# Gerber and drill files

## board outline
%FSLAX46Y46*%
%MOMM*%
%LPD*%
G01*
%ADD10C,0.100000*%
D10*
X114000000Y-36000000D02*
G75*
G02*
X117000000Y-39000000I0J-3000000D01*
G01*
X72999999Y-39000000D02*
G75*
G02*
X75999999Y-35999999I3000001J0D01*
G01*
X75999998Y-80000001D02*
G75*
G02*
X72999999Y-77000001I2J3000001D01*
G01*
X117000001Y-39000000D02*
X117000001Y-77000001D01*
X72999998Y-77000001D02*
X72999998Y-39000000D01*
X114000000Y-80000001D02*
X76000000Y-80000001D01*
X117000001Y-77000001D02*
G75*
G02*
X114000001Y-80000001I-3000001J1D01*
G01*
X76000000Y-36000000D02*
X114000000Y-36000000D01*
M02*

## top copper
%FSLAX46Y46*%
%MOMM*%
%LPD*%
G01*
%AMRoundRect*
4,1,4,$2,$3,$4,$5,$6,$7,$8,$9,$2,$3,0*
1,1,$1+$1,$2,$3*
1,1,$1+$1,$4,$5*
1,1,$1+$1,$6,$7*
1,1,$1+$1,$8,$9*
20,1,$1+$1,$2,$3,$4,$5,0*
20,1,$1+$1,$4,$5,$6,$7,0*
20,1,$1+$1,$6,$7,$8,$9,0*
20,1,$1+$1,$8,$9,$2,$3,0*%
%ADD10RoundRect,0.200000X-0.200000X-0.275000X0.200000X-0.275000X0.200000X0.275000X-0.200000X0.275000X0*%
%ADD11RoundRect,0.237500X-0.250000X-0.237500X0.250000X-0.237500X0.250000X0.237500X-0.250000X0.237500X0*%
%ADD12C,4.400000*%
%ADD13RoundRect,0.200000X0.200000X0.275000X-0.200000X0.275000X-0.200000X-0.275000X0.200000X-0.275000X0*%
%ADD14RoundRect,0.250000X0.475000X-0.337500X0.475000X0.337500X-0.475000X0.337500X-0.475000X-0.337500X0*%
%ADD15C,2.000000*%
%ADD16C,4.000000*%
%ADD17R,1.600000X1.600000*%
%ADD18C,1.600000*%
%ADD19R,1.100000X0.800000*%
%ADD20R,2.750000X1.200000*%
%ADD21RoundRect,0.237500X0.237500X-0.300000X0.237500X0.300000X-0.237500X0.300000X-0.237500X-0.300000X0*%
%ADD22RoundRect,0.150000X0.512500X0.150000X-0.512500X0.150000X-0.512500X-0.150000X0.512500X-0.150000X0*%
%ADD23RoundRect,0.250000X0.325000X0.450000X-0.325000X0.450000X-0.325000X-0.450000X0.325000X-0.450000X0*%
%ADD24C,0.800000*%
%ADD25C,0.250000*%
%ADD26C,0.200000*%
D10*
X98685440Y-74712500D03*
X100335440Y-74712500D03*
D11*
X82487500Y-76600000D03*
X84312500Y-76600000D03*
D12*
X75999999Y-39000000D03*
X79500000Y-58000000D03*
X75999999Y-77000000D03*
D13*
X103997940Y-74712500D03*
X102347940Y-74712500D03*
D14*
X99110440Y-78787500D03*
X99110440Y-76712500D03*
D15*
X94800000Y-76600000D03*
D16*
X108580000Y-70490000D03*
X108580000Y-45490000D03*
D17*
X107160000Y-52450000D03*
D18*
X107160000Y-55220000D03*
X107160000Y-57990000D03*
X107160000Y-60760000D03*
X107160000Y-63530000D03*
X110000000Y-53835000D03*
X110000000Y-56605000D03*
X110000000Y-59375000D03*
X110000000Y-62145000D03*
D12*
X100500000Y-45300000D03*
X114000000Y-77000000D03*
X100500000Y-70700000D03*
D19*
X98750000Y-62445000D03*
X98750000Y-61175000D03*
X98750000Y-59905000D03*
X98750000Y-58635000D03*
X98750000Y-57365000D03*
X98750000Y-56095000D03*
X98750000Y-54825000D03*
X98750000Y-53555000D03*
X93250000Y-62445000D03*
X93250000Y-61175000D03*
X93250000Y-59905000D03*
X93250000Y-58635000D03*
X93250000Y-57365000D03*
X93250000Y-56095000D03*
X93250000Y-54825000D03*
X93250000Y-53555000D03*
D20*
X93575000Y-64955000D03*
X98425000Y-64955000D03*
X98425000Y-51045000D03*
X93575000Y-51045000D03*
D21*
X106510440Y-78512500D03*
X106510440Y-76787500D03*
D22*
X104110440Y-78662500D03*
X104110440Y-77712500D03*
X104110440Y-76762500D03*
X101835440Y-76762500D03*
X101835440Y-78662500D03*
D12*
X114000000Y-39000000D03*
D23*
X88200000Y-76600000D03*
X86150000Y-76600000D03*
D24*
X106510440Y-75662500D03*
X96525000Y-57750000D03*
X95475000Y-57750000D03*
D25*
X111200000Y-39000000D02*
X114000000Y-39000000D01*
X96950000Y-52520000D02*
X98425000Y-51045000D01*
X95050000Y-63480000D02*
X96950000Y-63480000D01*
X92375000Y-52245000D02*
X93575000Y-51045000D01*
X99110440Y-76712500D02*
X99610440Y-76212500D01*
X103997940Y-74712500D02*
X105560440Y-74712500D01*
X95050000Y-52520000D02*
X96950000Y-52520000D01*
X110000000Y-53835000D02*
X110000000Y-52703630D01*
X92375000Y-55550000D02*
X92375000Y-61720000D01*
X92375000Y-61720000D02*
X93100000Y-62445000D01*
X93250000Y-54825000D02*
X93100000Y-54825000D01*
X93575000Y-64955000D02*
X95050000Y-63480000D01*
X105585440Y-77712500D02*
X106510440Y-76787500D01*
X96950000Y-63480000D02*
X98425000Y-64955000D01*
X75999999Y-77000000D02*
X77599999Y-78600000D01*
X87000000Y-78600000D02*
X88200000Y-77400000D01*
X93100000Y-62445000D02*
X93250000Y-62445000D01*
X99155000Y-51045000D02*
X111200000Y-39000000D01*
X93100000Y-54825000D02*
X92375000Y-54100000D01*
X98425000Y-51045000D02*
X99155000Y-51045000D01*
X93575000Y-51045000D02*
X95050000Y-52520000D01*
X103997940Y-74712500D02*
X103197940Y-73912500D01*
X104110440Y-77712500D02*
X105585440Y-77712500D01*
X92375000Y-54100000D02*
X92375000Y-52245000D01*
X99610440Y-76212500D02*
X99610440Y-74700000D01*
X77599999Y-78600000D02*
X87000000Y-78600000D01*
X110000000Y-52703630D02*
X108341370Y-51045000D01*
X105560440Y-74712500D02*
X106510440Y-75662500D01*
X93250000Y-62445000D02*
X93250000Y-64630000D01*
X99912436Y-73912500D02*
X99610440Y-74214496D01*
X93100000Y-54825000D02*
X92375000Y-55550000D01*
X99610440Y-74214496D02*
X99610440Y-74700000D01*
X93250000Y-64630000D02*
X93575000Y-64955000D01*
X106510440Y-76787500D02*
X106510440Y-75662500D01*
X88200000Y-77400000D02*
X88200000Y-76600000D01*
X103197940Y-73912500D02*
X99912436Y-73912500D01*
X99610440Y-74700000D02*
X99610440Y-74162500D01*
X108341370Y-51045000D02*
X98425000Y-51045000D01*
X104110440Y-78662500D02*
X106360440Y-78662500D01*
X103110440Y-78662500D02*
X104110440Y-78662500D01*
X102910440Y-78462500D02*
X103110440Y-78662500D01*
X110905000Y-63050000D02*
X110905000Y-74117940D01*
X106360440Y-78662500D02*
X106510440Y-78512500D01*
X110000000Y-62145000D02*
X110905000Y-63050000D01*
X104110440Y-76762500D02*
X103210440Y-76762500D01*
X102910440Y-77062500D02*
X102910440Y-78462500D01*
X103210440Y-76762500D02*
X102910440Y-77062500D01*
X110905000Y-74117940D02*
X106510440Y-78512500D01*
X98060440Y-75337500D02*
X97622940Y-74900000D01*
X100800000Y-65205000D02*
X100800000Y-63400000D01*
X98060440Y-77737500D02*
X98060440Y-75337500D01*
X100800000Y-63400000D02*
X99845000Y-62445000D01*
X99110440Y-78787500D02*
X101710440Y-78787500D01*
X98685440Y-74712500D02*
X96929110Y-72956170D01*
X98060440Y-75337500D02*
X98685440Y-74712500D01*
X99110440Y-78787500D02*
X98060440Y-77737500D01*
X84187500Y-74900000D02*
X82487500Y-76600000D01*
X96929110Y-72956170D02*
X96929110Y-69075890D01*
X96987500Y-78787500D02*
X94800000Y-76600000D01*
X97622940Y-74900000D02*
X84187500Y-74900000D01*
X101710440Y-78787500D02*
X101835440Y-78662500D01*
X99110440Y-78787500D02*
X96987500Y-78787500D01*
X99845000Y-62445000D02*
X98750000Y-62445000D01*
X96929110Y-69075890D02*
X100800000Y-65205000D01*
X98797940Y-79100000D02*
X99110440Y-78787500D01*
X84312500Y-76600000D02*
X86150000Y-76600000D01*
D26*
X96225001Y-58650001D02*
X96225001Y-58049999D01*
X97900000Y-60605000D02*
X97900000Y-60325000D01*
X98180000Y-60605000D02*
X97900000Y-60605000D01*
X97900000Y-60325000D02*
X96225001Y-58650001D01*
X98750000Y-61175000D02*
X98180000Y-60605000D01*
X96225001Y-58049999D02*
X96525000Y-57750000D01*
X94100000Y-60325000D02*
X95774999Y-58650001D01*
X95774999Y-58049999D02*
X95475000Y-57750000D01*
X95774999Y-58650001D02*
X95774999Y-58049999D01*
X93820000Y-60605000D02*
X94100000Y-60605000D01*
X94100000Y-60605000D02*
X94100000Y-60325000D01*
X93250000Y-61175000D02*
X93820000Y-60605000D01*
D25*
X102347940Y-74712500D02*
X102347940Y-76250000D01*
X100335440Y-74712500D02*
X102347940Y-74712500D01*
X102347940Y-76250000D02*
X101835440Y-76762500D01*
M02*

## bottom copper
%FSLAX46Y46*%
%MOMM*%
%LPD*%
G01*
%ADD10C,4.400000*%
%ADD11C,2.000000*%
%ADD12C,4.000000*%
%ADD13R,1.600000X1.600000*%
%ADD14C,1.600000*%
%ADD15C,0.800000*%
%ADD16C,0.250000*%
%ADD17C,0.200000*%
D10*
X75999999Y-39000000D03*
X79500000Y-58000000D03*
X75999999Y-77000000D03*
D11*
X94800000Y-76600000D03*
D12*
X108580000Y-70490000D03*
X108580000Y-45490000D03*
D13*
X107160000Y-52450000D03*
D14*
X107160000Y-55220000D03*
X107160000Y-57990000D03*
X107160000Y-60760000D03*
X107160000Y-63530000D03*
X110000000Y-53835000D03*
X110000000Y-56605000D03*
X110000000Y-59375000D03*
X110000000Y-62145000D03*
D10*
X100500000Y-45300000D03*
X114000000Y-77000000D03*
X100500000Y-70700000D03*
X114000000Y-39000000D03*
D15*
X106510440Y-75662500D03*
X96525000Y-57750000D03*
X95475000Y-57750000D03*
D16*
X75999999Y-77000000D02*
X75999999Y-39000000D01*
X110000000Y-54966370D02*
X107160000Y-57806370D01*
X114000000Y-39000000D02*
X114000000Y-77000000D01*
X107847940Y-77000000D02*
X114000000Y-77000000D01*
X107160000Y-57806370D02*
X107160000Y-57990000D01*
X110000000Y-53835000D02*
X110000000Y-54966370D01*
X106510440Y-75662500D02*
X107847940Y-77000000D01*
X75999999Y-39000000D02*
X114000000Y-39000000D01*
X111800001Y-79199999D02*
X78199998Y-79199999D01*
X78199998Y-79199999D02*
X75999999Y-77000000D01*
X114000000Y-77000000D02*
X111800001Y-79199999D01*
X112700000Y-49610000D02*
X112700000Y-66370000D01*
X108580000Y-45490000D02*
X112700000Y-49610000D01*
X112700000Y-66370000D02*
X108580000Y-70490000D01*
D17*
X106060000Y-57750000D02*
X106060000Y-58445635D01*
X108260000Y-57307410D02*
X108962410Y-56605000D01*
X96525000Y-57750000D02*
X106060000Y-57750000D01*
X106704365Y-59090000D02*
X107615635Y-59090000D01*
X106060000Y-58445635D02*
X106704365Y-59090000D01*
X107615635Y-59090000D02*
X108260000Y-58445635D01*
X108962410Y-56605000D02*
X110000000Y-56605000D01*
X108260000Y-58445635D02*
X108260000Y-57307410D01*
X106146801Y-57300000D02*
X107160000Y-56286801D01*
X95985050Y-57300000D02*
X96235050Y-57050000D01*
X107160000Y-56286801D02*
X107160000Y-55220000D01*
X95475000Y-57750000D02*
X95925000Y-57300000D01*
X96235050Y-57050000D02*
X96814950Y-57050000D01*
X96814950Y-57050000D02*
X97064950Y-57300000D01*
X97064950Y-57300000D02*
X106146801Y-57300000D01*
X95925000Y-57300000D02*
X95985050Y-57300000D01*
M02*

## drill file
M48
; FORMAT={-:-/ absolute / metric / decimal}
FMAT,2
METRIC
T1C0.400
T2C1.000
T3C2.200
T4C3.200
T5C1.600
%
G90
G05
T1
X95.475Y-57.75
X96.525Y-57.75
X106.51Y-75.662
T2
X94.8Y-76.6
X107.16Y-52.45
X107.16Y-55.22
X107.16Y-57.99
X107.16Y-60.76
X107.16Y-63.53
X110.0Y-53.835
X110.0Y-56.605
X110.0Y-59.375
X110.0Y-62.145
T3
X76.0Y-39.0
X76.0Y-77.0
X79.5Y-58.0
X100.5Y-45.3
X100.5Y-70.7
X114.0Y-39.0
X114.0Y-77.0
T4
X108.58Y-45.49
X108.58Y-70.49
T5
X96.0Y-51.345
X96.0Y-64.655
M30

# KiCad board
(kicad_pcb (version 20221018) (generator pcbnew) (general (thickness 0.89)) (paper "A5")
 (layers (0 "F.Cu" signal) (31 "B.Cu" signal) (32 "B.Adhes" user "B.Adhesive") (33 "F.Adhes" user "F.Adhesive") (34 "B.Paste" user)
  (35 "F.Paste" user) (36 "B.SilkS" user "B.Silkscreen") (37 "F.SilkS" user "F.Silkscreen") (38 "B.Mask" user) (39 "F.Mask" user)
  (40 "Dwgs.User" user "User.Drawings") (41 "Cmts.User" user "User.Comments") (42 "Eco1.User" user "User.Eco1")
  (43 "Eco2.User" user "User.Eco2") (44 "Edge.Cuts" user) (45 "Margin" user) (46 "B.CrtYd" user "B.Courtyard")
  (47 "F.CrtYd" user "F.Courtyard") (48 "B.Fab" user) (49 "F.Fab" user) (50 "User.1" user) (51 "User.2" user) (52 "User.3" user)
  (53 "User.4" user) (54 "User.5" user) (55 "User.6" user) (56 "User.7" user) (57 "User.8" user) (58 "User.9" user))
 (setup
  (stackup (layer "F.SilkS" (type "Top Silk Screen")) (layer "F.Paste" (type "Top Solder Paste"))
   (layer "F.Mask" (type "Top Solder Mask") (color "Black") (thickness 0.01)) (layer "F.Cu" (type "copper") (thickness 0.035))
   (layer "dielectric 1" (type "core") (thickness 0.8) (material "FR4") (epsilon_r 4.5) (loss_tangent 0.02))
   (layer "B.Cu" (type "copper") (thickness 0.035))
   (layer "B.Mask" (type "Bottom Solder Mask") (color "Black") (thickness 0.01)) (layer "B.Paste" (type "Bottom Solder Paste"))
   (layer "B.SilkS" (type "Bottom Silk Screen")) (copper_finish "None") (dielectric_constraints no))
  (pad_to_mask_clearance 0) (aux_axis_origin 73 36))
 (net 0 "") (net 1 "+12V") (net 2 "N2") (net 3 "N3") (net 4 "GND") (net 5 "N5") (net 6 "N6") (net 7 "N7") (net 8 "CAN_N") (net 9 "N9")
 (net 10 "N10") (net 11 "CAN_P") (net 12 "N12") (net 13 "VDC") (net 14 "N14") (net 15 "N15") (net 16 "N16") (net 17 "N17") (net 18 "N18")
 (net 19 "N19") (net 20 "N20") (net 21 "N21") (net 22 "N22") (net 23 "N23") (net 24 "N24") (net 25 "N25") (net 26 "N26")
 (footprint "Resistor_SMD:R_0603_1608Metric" (layer "F.Cu") (at 99.51044 74.7125)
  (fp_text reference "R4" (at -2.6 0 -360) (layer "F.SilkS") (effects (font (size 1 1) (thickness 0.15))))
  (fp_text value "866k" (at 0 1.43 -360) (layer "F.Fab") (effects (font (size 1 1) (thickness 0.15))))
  (pad "1" smd roundrect (at -0.825 0) (size 0.8 0.95) (layers "F.Cu" "F.Paste" "F.Mask") (roundrect_rratio 0.25) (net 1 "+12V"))
  (pad "2" smd roundrect (at 0.825 0) (size 0.8 0.95) (layers "F.Cu" "F.Paste" "F.Mask") (roundrect_rratio 0.25) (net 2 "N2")))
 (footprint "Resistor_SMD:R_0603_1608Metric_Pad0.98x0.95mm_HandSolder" (layer "F.Cu") (at 83.4 76.6)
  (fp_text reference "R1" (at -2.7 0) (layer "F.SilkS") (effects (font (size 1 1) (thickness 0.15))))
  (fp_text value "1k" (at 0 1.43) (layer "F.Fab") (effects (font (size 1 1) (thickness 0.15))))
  (pad "1" smd roundrect (at -0.9125 0) (size 0.975 0.95) (layers "F.Cu" "F.Paste" "F.Mask") (roundrect_rratio 0.25) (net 1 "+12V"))
  (pad "2" smd roundrect (at 0.9125 0) (size 0.975 0.95) (layers "F.Cu" "F.Paste" "F.Mask") (roundrect_rratio 0.25) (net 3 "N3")))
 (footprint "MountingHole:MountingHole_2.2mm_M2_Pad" (layer "F.Cu") (at 75.999999 39)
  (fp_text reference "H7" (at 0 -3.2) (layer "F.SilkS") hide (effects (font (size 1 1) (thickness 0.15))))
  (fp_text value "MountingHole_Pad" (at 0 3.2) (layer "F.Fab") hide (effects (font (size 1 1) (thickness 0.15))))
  (pad "1" thru_hole circle (at 0 0) (size 4.4 4.4) (drill 2.2) (layers "*.Cu" "*.Mask") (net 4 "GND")))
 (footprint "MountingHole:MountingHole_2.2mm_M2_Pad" (layer "F.Cu") (at 79.5 58 90)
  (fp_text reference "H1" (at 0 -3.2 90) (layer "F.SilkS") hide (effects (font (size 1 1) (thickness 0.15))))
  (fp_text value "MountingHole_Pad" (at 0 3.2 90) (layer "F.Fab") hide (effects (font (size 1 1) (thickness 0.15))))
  (pad "1" thru_hole circle (at 0 0 90) (size 4.4 4.4) (drill 2.2) (layers "*.Cu" "*.Mask") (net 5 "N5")))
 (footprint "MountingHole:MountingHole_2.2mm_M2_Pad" (layer "F.Cu") (at 75.999999 77)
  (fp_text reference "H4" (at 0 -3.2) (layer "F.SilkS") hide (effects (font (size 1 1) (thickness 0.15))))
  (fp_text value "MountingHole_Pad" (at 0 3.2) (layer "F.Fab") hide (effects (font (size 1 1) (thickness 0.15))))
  (pad "1" thru_hole circle (at 0 0) (size 4.4 4.4) (drill 2.2) (layers "*.Cu" "*.Mask") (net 4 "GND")))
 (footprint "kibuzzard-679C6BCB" (layer "F.Cu") (at 90.8 76.6)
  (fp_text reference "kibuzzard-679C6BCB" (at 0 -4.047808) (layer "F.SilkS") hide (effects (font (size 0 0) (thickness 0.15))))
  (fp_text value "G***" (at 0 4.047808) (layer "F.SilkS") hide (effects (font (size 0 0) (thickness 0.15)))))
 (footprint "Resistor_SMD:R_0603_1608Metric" (layer "F.Cu") (at 103.17294 74.7125 180)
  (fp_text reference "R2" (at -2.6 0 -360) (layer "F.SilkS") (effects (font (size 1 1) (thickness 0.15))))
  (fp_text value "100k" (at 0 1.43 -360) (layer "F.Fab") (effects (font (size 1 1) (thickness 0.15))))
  (pad "1" smd roundrect (at -0.825 0 180) (size 0.8 0.95) (layers "F.Cu" "F.Paste" "F.Mask") (roundrect_rratio 0.25) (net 4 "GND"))
  (pad "2" smd roundrect (at 0.825 0 180) (size 0.8 0.95) (layers "F.Cu" "F.Paste" "F.Mask") (roundrect_rratio 0.25) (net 2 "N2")))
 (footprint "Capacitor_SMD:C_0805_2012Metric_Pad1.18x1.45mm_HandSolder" (layer "F.Cu") (at 99.11044 77.75 90)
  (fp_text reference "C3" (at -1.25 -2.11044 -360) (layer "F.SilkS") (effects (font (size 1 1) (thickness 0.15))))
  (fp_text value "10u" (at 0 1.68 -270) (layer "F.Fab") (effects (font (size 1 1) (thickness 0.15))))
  (pad "1" smd roundrect (at -1.0375 0 90) (size 1.175 1.45) (layers "F.Cu" "F.Paste" "F.Mask") (roundrect_rratio 0.2127659574)
   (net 1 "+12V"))
  (pad "2" smd roundrect (at 1.0375 0 90) (size 1.175 1.45) (layers "F.Cu" "F.Paste" "F.Mask") (roundrect_rratio 0.2127659574) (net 4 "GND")))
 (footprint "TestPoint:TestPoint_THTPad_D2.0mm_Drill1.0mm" (layer "F.Cu") (at 94.8 76.6)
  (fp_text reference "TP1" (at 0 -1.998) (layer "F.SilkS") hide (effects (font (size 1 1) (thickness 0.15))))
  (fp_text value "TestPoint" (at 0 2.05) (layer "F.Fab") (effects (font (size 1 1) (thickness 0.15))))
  (pad "1" thru_hole circle (at 0 0) (size 2 2) (drill 1) (layers "*.Cu" "*.Mask") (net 1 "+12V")))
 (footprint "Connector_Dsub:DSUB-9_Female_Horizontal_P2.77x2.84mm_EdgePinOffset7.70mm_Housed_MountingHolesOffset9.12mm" (layer "F.Cu")
  (at 107.16 52.45 90)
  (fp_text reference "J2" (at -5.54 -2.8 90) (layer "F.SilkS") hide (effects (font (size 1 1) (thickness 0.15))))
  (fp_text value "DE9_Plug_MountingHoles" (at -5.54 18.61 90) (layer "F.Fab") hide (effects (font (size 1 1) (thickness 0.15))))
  (pad "0" thru_hole circle (at -18.04 1.42 90) (size 4 4) (drill 3.2) (layers "*.Cu" "*.Mask") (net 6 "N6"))
  (pad "0" thru_hole circle (at 6.96 1.42 90) (size 4 4) (drill 3.2) (layers "*.Cu" "*.Mask") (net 6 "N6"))
  (pad "1" thru_hole rect (at 0 0 90) (size 1.6 1.6) (drill 1) (layers "*.Cu" "*.Mask") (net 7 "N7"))
  (pad "2" thru_hole circle (at -2.77 0 90) (size 1.6 1.6) (drill 1) (layers "*.Cu" "*.Mask") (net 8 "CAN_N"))
  (pad "3" thru_hole circle (at -5.54 0 90) (size 1.6 1.6) (drill 1) (layers "*.Cu" "*.Mask") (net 4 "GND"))
  (pad "4" thru_hole circle (at -8.31 0 90) (size 1.6 1.6) (drill 1) (layers "*.Cu" "*.Mask") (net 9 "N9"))
  (pad "5" thru_hole circle (at -11.08 0 90) (size 1.6 1.6) (drill 1) (layers "*.Cu" "*.Mask") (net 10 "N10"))
  (pad "6" thru_hole circle (at -1.385 2.84 90) (size 1.6 1.6) (drill 1) (layers "*.Cu" "*.Mask") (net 4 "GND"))
  (pad "7" thru_hole circle (at -4.155 2.84 90) (size 1.6 1.6) (drill 1) (layers "*.Cu" "*.Mask") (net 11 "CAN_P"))
  (pad "8" thru_hole circle (at -6.925 2.84 90) (size 1.6 1.6) (drill 1) (layers "*.Cu" "*.Mask") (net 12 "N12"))
  (pad "9" thru_hole circle (at -9.695 2.84 90) (size 1.6 1.6) (drill 1) (layers "*.Cu" "*.Mask") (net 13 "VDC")))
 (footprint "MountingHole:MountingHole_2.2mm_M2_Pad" (layer "F.Cu") (at 100.5 45.3 90)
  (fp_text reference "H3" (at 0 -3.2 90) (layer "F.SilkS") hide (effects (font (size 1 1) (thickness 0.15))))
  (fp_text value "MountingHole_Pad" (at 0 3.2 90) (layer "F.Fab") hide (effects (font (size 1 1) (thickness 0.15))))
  (pad "1" thru_hole circle (at 0 0 90) (size 4.4 4.4) (drill 2.2) (layers "*.Cu" "*.Mask") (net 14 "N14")))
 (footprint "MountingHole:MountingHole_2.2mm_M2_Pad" (layer "F.Cu") (at 114 77)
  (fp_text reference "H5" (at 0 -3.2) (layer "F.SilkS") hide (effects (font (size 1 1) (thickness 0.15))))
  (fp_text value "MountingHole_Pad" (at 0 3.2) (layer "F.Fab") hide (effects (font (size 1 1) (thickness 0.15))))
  (pad "1" thru_hole circle (at 0 0) (size 4.4 4.4) (drill 2.2) (layers "*.Cu" "*.Mask") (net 4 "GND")))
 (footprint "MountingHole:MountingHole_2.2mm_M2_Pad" (layer "F.Cu") (at 100.5 70.7 90)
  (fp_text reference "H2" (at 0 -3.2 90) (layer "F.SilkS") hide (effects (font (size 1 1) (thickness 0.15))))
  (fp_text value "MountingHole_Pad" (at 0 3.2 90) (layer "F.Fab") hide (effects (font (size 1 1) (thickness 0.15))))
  (pad "1" thru_hole circle (at 0 0 90) (size 4.4 4.4) (drill 2.2) (layers "*.Cu" "*.Mask") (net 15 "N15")))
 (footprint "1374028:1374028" (layer "F.Cu") (at 96 58 90)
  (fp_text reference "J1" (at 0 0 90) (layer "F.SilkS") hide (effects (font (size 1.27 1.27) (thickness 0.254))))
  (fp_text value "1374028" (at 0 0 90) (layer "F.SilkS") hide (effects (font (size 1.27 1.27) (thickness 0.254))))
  (pad "" np_thru_hole circle (at -6.655 0 90) (size 1.6 1.6) (drill 1.6) (layers "*.Cu" "*.Mask"))
  (pad "" np_thru_hole circle (at 6.655 0 90) (size 1.6 1.6) (drill 1.6) (layers "*.Cu" "*.Mask"))
  (pad "A1" smd rect (at -4.445 2.75 90) (size 0.8 1.1) (layers "F.Cu" "F.Paste" "F.Mask") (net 1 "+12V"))
  (pad "A2" smd rect (at -3.175 2.75 90) (size 0.8 1.1) (layers "F.Cu" "F.Paste" "F.Mask") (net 11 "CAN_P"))
  (pad "A3" smd rect (at -1.905 2.75 90) (size 0.8 1.1) (layers "F.Cu" "F.Paste" "F.Mask") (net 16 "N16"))
  (pad "A4" smd rect (at -0.635 2.75 90) (size 0.8 1.1) (layers "F.Cu" "F.Paste" "F.Mask") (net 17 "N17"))
  (pad "A5" smd rect (at 0.635 2.75 90) (size 0.8 1.1) (layers "F.Cu" "F.Paste" "F.Mask") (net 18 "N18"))
  (pad "A6" smd rect (at 1.905 2.75 90) (size 0.8 1.1) (layers "F.Cu" "F.Paste" "F.Mask") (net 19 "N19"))
  (pad "A7" smd rect (at 3.175 2.75 90) (size 0.8 1.1) (layers "F.Cu" "F.Paste" "F.Mask") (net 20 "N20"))
  (pad "A8" smd rect (at 4.445 2.75 90) (size 0.8 1.1) (layers "F.Cu" "F.Paste" "F.Mask") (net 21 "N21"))
  (pad "B1" smd rect (at -4.445 -2.75 90) (size 0.8 1.1) (layers "F.Cu" "F.Paste" "F.Mask") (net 4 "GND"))
  (pad "B2" smd rect (at -3.175 -2.75 90) (size 0.8 1.1) (layers "F.Cu" "F.Paste" "F.Mask") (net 8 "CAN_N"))
  (pad "B3" smd rect (at -1.905 -2.75 90) (size 0.8 1.1) (layers "F.Cu" "F.Paste" "F.Mask") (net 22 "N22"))
  (pad "B4" smd rect (at -0.635 -2.75 90) (size 0.8 1.1) (layers "F.Cu" "F.Paste" "F.Mask") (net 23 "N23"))
  (pad "B5" smd rect (at 0.635 -2.75 90) (size 0.8 1.1) (layers "F.Cu" "F.Paste" "F.Mask") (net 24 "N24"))
  (pad "B6" smd rect (at 1.905 -2.75 90) (size 0.8 1.1) (layers "F.Cu" "F.Paste" "F.Mask") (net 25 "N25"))
  (pad "B7" smd rect (at 3.175 -2.75 90) (size 0.8 1.1) (layers "F.Cu" "F.Paste" "F.Mask") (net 4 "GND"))
  (pad "B8" smd rect (at 4.445 -2.75 90) (size 0.8 1.1) (layers "F.Cu" "F.Paste" "F.Mask") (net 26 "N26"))
  (pad "MP1" smd rect (at -6.955 -2.425 90) (size 1.2 2.75) (layers "F.Cu" "F.Paste" "F.Mask") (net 4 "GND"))
  (pad "MP2" smd rect (at -6.955 2.425 90) (size 1.2 2.75) (layers "F.Cu" "F.Paste" "F.Mask") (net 4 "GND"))
  (pad "MP3" smd rect (at 6.955 2.425 90) (size 1.2 2.75) (layers "F.Cu" "F.Paste" "F.Mask") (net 4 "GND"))
  (pad "MP4" smd rect (at 6.955 -2.425 90) (size 1.2 2.75) (layers "F.Cu" "F.Paste" "F.Mask") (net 4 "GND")))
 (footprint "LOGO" (layer "F.Cu") (at 105.25 39)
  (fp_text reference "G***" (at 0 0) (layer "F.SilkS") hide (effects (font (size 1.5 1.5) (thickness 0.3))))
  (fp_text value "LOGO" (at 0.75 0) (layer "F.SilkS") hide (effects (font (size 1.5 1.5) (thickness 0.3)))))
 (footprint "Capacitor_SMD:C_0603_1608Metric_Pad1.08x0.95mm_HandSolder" (layer "F.Cu") (at 106.51044 77.65 90)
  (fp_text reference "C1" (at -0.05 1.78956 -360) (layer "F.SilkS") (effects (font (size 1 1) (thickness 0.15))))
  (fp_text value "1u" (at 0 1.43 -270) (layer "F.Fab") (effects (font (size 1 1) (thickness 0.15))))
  (pad "1" smd roundrect (at -0.8625 0 90) (size 1.075 0.95) (layers "F.Cu" "F.Paste" "F.Mask") (roundrect_rratio 0.25) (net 13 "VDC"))
  (pad "2" smd roundrect (at 0.8625 0 90) (size 1.075 0.95) (layers "F.Cu" "F.Paste" "F.Mask") (roundrect_rratio 0.25) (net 4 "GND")))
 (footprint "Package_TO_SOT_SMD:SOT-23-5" (layer "F.Cu") (at 102.97294 77.7125 180)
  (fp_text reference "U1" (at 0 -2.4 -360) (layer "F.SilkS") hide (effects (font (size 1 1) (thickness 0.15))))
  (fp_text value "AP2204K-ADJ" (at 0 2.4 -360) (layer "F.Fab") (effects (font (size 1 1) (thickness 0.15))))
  (pad "1" smd roundrect (at -1.1375 -0.95 180) (size 1.325 0.6) (layers "F.Cu" "F.Paste" "F.Mask") (roundrect_rratio 0.25) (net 13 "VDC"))
  (pad "2" smd roundrect (at -1.1375 0 180) (size 1.325 0.6) (layers "F.Cu" "F.Paste" "F.Mask") (roundrect_rratio 0.25) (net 4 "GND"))
  (pad "3" smd roundrect (at -1.1375 0.95 180) (size 1.325 0.6) (layers "F.Cu" "F.Paste" "F.Mask") (roundrect_rratio 0.25) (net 13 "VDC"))
  (pad "4" smd roundrect (at 1.1375 0.95 180) (size 1.325 0.6) (layers "F.Cu" "F.Paste" "F.Mask") (roundrect_rratio 0.25) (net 2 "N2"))
  (pad "5" smd roundrect (at 1.1375 -0.95 180) (size 1.325 0.6) (layers "F.Cu" "F.Paste" "F.Mask") (roundrect_rratio 0.25) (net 1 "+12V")))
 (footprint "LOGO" (layer "F.Cu") (at 92.25 39)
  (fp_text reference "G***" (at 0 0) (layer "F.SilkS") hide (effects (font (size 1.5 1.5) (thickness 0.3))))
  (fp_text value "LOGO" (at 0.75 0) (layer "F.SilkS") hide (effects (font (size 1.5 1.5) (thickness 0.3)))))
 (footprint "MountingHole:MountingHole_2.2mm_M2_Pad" (layer "F.Cu") (at 114 39)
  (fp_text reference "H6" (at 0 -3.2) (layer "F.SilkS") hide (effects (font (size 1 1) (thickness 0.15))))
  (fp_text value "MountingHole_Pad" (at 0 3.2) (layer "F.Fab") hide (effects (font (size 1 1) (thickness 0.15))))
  (pad "1" thru_hole circle (at 0 0) (size 4.4 4.4) (drill 2.2) (layers "*.Cu" "*.Mask") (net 4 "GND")))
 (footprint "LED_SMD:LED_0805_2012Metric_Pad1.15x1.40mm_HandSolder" (layer "F.Cu") (at 87.175 76.6 180)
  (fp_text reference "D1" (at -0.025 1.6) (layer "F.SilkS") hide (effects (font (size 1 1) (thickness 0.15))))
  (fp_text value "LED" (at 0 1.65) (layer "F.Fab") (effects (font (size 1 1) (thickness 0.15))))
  (pad "1" smd roundrect (at -1.025 0 180) (size 1.15 1.4) (layers "F.Cu" "F.Paste" "F.Mask") (roundrect_rratio 0.2173913043) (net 4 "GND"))
  (pad "2" smd roundrect (at 1.025 0 180) (size 1.15 1.4) (layers "F.Cu" "F.Paste" "F.Mask") (roundrect_rratio 0.2173913043) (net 3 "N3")))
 (gr_arc (start 114 36) (mid 116.12132 36.87868) (end 117 39) (stroke (width 0.1) (type default)) (layer "Edge.Cuts"))
 (gr_arc (start 72.999999 39) (mid 73.878679 36.87868) (end 75.999999 36) (stroke (width 0.1) (type default)) (layer "Edge.Cuts"))
 (gr_arc (start 75.999998 80.000001) (mid 73.878678 79.121321) (end 72.999998 77.000001) (stroke (width 0.1) (type default))
  (layer "Edge.Cuts"))
 (gr_line (start 117.000001 39) (end 117.000001 77.000001) (stroke (width 0.1) (type default)) (layer "Edge.Cuts"))
 (gr_line (start 72.999998 77.000001) (end 72.999998 39) (stroke (width 0.1) (type default)) (layer "Edge.Cuts"))
 (gr_line (start 114 80.000001) (end 76 80.000001) (stroke (width 0.1) (type default)) (layer "Edge.Cuts"))
 (gr_arc (start 117.000001 77.000001) (mid 116.121321 79.121321) (end 114.000001 80.000001) (stroke (width 0.1) (type default))
  (layer "Edge.Cuts"))
 (gr_line (start 76 36) (end 114 36) (stroke (width 0.1) (type default)) (layer "Edge.Cuts"))
 (segment (start 111.2 39) (end 114 39) (width 0.25) (layer "F.Cu") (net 4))
 (segment (start 96.95 52.52) (end 98.425 51.045) (width 0.25) (layer "F.Cu") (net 4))
 (segment (start 95.05 63.48) (end 96.95 63.48) (width 0.25) (layer "F.Cu") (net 4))
 (segment (start 92.375 52.245) (end 93.575 51.045) (width 0.25) (layer "F.Cu") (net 4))
 (segment (start 99.11044 76.7125) (end 99.61044 76.2125) (width 0.25) (layer "F.Cu") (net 4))
 (segment (start 103.99794 74.7125) (end 105.56044 74.7125) (width 0.25) (layer "F.Cu") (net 4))
 (segment (start 95.05 52.52) (end 96.95 52.52) (width 0.25) (layer "F.Cu") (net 4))
 (segment (start 110 53.835) (end 110 52.70363) (width 0.25) (layer "F.Cu") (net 4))
 (segment (start 92.375 55.55) (end 92.375 61.72) (width 0.25) (layer "F.Cu") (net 4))
 (segment (start 92.375 61.72) (end 93.1 62.445) (width 0.25) (layer "F.Cu") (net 4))
 (segment (start 93.25 54.825) (end 93.1 54.825) (width 0.25) (layer "F.Cu") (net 4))
 (segment (start 93.575 64.955) (end 95.05 63.48) (width 0.25) (layer "F.Cu") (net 4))
 (segment (start 105.58544 77.7125) (end 106.51044 76.7875) (width 0.25) (layer "F.Cu") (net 4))
 (segment (start 96.95 63.48) (end 98.425 64.955) (width 0.25) (layer "F.Cu") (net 4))
 (segment (start 75.999999 77) (end 77.599999 78.6) (width 0.25) (layer "F.Cu") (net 4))
 (segment (start 87 78.6) (end 88.2 77.4) (width 0.25) (layer "F.Cu") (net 4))
 (segment (start 93.1 62.445) (end 93.25 62.445) (width 0.25) (layer "F.Cu") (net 4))
 (segment (start 99.155 51.045) (end 111.2 39) (width 0.25) (layer "F.Cu") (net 4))
 (segment (start 93.1 54.825) (end 92.375 54.1) (width 0.25) (layer "F.Cu") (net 4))
 (segment (start 98.425 51.045) (end 99.155 51.045) (width 0.25) (layer "F.Cu") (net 4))
 (segment (start 93.575 51.045) (end 95.05 52.52) (width 0.25) (layer "F.Cu") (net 4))
 (segment (start 103.99794 74.7125) (end 103.19794 73.9125) (width 0.25) (layer "F.Cu") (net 4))
 (segment (start 104.11044 77.7125) (end 105.58544 77.7125) (width 0.25) (layer "F.Cu") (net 4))
 (segment (start 92.375 54.1) (end 92.375 52.245) (width 0.25) (layer "F.Cu") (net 4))
 (segment (start 99.61044 76.2125) (end 99.61044 74.7) (width 0.25) (layer "F.Cu") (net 4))
 (segment (start 77.599999 78.6) (end 87 78.6) (width 0.25) (layer "F.Cu") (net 4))
 (segment (start 110 52.70363) (end 108.34137 51.045) (width 0.25) (layer "F.Cu") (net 4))
 (segment (start 105.56044 74.7125) (end 106.51044 75.6625) (width 0.25) (layer "F.Cu") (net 4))
 (segment (start 93.25 62.445) (end 93.25 64.63) (width 0.25) (layer "F.Cu") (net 4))
 (segment (start 99.912436 73.9125) (end 99.61044 74.214496) (width 0.25) (layer "F.Cu") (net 4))
 (segment (start 93.1 54.825) (end 92.375 55.55) (width 0.25) (layer "F.Cu") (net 4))
 (segment (start 99.61044 74.214496) (end 99.61044 74.7) (width 0.25) (layer "F.Cu") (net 4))
 (segment (start 93.25 64.63) (end 93.575 64.955) (width 0.25) (layer "F.Cu") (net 4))
 (segment (start 106.51044 76.7875) (end 106.51044 75.6625) (width 0.25) (layer "F.Cu") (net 4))
 (segment (start 88.2 77.4) (end 88.2 76.6) (width 0.25) (layer "F.Cu") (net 4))
 (segment (start 103.19794 73.9125) (end 99.912436 73.9125) (width 0.25) (layer "F.Cu") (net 4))
 (segment (start 99.61044 74.7) (end 99.61044 74.1625) (width 0.25) (layer "F.Cu") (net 4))
 (segment (start 108.34137 51.045) (end 98.425 51.045) (width 0.25) (layer "F.Cu") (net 4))
 (via (at 106.51044 75.6625) (size 0.8) (drill 0.4) (layers "F.Cu" "B.Cu") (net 4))
 (segment (start 75.999999 77) (end 75.999999 39) (width 0.25) (layer "B.Cu") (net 4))
 (segment (start 110 54.96637) (end 107.16 57.80637) (width 0.25) (layer "B.Cu") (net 4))
 (segment (start 114 39) (end 114 77) (width 0.25) (layer "B.Cu") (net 4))
 (segment (start 107.84794 77) (end 114 77) (width 0.25) (layer "B.Cu") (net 4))
 (segment (start 107.16 57.80637) (end 107.16 57.99) (width 0.25) (layer "B.Cu") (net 4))
 (segment (start 110 53.835) (end 110 54.96637) (width 0.25) (layer "B.Cu") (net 4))
 (segment (start 106.51044 75.6625) (end 107.84794 77) (width 0.25) (layer "B.Cu") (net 4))
 (segment (start 75.999999 39) (end 114 39) (width 0.25) (layer "B.Cu") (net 4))
 (segment (start 111.800001 79.199999) (end 78.199998 79.199999) (width 0.25) (layer "B.Cu") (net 4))
 (segment (start 78.199998 79.199999) (end 75.999999 77) (width 0.25) (layer "B.Cu") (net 4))
 (segment (start 114 77) (end 111.800001 79.199999) (width 0.25) (layer "B.Cu") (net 4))
 (segment (start 104.11044 78.6625) (end 106.36044 78.6625) (width 0.25) (layer "F.Cu") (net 13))
 (segment (start 103.11044 78.6625) (end 104.11044 78.6625) (width 0.25) (layer "F.Cu") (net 13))
 (segment (start 102.91044 78.4625) (end 103.11044 78.6625) (width 0.25) (layer "F.Cu") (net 13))
 (segment (start 110.905 63.05) (end 110.905 74.11794) (width 0.25) (layer "F.Cu") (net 13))
 (segment (start 106.36044 78.6625) (end 106.51044 78.5125) (width 0.25) (layer "F.Cu") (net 13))
 (segment (start 110 62.145) (end 110.905 63.05) (width 0.25) (layer "F.Cu") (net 13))
 (segment (start 104.11044 76.7625) (end 103.21044 76.7625) (width 0.25) (layer "F.Cu") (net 13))
 (segment (start 102.91044 77.0625) (end 102.91044 78.4625) (width 0.25) (layer "F.Cu") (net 13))
 (segment (start 103.21044 76.7625) (end 102.91044 77.0625) (width 0.25) (layer "F.Cu") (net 13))
 (segment (start 110.905 74.11794) (end 106.51044 78.5125) (width 0.25) (layer "F.Cu") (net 13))
 (segment (start 98.06044 75.3375) (end 97.62294 74.9) (width 0.25) (layer "F.Cu") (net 1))
 (segment (start 100.8 65.205) (end 100.8 63.4) (width 0.25) (layer "F.Cu") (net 1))
 (segment (start 98.06044 77.7375) (end 98.06044 75.3375) (width 0.25) (layer "F.Cu") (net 1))
 (segment (start 100.8 63.4) (end 99.845 62.445) (width 0.25) (layer "F.Cu") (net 1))
 (segment (start 99.11044 78.7875) (end 101.71044 78.7875) (width 0.25) (layer "F.Cu") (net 1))
 (segment (start 98.68544 74.7125) (end 96.92911 72.95617) (width 0.25) (layer "F.Cu") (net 1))
 (segment (start 98.06044 75.3375) (end 98.68544 74.7125) (width 0.25) (layer "F.Cu") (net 1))
 (segment (start 99.11044 78.7875) (end 98.06044 77.7375) (width 0.25) (layer "F.Cu") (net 1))
 (segment (start 84.1875 74.9) (end 82.4875 76.6) (width 0.25) (layer "F.Cu") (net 1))
 (segment (start 96.92911 72.95617) (end 96.92911 69.07589) (width 0.25) (layer "F.Cu") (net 1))
 (segment (start 96.9875 78.7875) (end 94.8 76.6) (width 0.25) (layer "F.Cu") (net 1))
 (segment (start 97.62294 74.9) (end 84.1875 74.9) (width 0.25) (layer "F.Cu") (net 1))
 (segment (start 101.71044 78.7875) (end 101.83544 78.6625) (width 0.25) (layer "F.Cu") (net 1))
 (segment (start 99.11044 78.7875) (end 96.9875 78.7875) (width 0.25) (layer "F.Cu") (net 1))
 (segment (start 99.845 62.445) (end 98.75 62.445) (width 0.25) (layer "F.Cu") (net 1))
 (segment (start 96.92911 69.07589) (end 100.8 65.205) (width 0.25) (layer "F.Cu") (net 1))
 (segment (start 98.79794 79.1) (end 99.11044 78.7875) (width 0.25) (layer "F.Cu") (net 1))
 (segment (start 84.3125 76.6) (end 86.15 76.6) (width 0.25) (layer "F.Cu") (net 3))
 (segment (start 112.7 49.61) (end 112.7 66.37) (width 0.25) (layer "B.Cu") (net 6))
 (segment (start 108.58 45.49) (end 112.7 49.61) (width 0.25) (layer "B.Cu") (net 6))
 (segment (start 112.7 66.37) (end 108.58 70.49) (width 0.25) (layer "B.Cu") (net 6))
 (segment (start 96.225001 58.650001) (end 96.225001 58.049999) (width 0.2) (layer "F.Cu") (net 11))
 (segment (start 97.9 60.605) (end 97.9 60.325) (width 0.2) (layer "F.Cu") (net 11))
 (segment (start 98.18 60.605) (end 97.9 60.605) (width 0.2) (layer "F.Cu") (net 11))
 (segment (start 97.9 60.325) (end 96.225001 58.650001) (width 0.2) (layer "F.Cu") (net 11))
 (segment (start 98.75 61.175) (end 98.18 60.605) (width 0.2) (layer "F.Cu") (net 11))
 (segment (start 96.225001 58.049999) (end 96.525 57.75) (width 0.2) (layer "F.Cu") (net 11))
 (via (at 96.525 57.75) (size 0.8) (drill 0.4) (layers "F.Cu" "B.Cu") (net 11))
 (segment (start 106.06 57.75) (end 106.06 58.445635) (width 0.2) (layer "B.Cu") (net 11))
 (segment (start 108.26 57.30741) (end 108.96241 56.605) (width 0.2) (layer "B.Cu") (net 11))
 (segment (start 96.525 57.75) (end 106.06 57.75) (width 0.2) (layer "B.Cu") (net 11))
 (segment (start 106.704365 59.09) (end 107.615635 59.09) (width 0.2) (layer "B.Cu") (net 11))
 (segment (start 106.06 58.445635) (end 106.704365 59.09) (width 0.2) (layer "B.Cu") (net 11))
 (segment (start 107.615635 59.09) (end 108.26 58.445635) (width 0.2) (layer "B.Cu") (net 11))
 (segment (start 108.96241 56.605) (end 110 56.605) (width 0.2) (layer "B.Cu") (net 11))
 (segment (start 108.26 58.445635) (end 108.26 57.30741) (width 0.2) (layer "B.Cu") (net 11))
 (segment (start 94.1 60.325) (end 95.774999 58.650001) (width 0.2) (layer "F.Cu") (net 8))
 (segment (start 95.774999 58.049999) (end 95.475 57.75) (width 0.2) (layer "F.Cu") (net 8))
 (segment (start 95.774999 58.650001) (end 95.774999 58.049999) (width 0.2) (layer "F.Cu") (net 8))
 (segment (start 93.82 60.605) (end 94.1 60.605) (width 0.2) (layer "F.Cu") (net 8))
 (segment (start 94.1 60.605) (end 94.1 60.325) (width 0.2) (layer "F.Cu") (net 8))
 (segment (start 93.25 61.175) (end 93.82 60.605) (width 0.2) (layer "F.Cu") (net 8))
 (via (at 95.475 57.75) (size 0.8) (drill 0.4) (layers "F.Cu" "B.Cu") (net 8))
 (segment (start 106.146801 57.3) (end 107.16 56.286801) (width 0.2) (layer "B.Cu") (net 8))
 (segment (start 95.98505 57.3) (end 96.23505 57.05) (width 0.2) (layer "B.Cu") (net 8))
 (segment (start 107.16 56.286801) (end 107.16 55.22) (width 0.2) (layer "B.Cu") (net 8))
 (segment (start 95.475 57.75) (end 95.925 57.3) (width 0.2) (layer "B.Cu") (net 8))
 (segment (start 96.23505 57.05) (end 96.81495 57.05) (width 0.2) (layer "B.Cu") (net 8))
 (segment (start 96.81495 57.05) (end 97.06495 57.3) (width 0.2) (layer "B.Cu") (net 8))
 (segment (start 97.06495 57.3) (end 106.146801 57.3) (width 0.2) (layer "B.Cu") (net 8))
 (segment (start 95.925 57.3) (end 95.98505 57.3) (width 0.2) (layer "B.Cu") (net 8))
 (segment (start 102.34794 74.7125) (end 102.34794 76.25) (width 0.25) (layer "F.Cu") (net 2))
 (segment (start 100.33544 74.7125) (end 102.34794 74.7125) (width 0.25) (layer "F.Cu") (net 2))
 (segment (start 102.34794 76.25) (end 101.83544 76.7625) (width 0.25) (layer "F.Cu") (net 2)))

